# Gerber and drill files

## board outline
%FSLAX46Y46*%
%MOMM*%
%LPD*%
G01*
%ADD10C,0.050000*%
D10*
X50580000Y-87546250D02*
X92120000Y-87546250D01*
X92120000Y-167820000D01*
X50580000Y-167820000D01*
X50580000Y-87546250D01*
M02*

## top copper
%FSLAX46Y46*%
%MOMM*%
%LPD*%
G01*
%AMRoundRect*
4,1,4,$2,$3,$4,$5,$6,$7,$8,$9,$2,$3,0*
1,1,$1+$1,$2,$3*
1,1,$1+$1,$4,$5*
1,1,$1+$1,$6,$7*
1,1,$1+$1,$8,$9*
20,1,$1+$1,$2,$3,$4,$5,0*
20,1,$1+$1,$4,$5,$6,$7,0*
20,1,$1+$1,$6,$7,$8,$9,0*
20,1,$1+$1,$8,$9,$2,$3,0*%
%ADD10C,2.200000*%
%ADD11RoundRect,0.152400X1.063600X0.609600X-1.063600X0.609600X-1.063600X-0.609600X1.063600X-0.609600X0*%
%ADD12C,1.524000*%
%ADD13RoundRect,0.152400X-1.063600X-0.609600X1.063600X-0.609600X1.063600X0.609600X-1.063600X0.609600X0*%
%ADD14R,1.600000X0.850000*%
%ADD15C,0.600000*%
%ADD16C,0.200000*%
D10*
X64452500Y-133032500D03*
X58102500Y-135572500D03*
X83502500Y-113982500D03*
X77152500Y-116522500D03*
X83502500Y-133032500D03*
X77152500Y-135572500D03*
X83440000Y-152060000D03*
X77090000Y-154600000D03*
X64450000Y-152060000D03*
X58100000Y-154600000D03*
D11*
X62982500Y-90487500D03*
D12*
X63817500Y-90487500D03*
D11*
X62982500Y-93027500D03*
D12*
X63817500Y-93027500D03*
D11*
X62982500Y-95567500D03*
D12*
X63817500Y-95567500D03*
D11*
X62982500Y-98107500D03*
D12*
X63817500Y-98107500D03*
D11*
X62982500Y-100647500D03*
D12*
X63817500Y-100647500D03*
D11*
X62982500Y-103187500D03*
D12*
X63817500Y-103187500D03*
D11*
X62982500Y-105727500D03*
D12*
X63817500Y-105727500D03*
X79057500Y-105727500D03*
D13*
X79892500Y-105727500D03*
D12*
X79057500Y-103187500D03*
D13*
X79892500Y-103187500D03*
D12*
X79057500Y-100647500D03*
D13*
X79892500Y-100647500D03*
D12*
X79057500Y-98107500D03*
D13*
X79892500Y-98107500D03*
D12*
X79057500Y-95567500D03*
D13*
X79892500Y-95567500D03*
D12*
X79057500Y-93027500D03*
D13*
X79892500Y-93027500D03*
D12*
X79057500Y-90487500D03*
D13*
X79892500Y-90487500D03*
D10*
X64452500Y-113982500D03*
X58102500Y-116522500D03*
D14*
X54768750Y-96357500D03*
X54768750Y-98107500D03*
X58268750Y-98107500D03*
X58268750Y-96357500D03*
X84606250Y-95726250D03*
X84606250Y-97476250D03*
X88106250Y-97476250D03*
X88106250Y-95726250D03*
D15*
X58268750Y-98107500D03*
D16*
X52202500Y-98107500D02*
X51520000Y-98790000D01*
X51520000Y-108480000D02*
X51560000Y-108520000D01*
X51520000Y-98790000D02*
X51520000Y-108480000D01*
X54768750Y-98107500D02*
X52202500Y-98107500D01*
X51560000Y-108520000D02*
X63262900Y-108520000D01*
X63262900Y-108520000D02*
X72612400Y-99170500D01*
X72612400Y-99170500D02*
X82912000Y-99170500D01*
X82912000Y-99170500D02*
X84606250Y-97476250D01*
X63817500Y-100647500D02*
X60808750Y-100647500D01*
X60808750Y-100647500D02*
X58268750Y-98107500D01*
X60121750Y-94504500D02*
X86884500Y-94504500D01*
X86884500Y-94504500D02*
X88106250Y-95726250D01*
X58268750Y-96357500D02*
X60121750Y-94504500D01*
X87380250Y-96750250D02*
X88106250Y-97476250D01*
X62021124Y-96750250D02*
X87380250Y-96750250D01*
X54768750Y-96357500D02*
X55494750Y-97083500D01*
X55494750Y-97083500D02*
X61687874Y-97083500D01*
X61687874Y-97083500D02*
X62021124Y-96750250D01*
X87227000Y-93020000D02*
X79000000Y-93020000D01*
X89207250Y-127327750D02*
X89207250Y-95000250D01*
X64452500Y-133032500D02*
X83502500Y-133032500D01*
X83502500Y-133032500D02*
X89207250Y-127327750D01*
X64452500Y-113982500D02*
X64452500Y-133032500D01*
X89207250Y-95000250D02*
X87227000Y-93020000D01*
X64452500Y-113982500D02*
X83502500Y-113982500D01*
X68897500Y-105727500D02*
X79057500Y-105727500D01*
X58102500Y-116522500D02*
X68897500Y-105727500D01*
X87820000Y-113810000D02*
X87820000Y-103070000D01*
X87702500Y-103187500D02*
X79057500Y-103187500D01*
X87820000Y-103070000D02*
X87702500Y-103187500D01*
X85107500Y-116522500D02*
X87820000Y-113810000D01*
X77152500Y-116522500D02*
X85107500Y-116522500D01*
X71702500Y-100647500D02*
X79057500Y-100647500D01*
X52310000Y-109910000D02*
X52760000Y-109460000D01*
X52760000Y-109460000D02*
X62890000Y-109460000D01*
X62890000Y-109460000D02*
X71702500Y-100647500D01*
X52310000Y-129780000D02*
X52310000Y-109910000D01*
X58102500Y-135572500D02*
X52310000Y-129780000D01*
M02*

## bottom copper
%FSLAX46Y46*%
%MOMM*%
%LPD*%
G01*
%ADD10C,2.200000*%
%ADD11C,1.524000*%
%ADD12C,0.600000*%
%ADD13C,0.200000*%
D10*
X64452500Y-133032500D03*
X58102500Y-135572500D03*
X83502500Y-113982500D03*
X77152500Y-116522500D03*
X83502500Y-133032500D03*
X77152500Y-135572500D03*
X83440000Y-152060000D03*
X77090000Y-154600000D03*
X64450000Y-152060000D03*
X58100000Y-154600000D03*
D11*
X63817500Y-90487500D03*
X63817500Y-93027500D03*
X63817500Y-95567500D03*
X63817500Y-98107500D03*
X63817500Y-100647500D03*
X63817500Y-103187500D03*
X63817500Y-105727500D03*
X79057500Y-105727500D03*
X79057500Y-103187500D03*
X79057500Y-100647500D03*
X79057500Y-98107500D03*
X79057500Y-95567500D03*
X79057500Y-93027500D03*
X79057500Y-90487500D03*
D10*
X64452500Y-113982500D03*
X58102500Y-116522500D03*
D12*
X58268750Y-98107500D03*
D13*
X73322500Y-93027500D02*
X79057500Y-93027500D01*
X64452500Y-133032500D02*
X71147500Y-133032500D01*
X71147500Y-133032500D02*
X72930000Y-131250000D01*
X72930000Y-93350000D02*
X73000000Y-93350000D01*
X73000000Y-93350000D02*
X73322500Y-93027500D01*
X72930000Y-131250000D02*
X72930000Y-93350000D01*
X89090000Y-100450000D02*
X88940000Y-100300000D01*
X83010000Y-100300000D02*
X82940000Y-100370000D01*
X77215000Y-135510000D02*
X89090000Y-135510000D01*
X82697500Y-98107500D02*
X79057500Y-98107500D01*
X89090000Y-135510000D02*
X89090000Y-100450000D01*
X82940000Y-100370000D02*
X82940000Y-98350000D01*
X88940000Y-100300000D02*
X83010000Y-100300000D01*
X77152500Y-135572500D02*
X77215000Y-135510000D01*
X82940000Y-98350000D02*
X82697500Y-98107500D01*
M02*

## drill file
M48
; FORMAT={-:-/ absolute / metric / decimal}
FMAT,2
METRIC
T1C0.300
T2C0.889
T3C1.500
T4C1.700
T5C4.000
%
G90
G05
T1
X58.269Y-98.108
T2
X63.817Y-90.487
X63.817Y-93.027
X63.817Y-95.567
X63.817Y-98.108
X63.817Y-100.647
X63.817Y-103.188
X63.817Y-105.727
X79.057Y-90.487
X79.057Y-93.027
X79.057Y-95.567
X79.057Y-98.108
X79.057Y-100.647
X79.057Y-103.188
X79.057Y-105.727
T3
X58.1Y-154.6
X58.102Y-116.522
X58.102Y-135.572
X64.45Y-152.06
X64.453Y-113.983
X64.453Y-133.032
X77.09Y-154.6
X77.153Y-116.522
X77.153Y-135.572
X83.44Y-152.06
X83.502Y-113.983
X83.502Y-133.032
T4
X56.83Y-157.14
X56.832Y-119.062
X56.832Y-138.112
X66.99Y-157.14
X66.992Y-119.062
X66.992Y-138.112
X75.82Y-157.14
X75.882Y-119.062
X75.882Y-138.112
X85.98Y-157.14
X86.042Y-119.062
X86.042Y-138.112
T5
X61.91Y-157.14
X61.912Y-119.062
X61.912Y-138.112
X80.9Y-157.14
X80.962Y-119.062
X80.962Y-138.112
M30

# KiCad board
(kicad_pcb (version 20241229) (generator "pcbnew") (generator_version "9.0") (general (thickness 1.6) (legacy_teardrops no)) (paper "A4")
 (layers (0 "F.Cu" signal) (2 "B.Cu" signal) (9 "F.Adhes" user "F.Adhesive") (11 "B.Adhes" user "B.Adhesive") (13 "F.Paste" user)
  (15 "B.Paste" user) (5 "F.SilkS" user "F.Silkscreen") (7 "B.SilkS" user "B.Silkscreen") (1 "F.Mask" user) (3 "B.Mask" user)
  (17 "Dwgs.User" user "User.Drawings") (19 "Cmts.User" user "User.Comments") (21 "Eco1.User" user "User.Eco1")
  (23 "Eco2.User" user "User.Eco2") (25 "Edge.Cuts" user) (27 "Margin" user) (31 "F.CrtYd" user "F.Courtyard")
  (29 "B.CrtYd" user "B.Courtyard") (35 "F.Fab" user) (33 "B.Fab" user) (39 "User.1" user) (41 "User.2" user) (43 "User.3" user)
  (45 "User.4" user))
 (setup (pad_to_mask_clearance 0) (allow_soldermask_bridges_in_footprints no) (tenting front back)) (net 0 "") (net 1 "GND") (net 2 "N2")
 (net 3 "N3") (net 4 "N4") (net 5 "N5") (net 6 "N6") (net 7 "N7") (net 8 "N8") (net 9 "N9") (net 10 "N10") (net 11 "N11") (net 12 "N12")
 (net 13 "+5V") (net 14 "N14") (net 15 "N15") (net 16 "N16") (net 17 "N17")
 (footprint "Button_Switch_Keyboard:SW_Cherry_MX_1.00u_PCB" (layer "F.Cu") (at 64.4525 133.0325)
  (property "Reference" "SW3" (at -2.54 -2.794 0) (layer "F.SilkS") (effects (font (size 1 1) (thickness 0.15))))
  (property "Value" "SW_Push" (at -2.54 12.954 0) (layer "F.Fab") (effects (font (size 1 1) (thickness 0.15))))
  (pad "" np_thru_hole circle (at -7.62 5.08) (size 1.7 1.7) (drill 1.7) (layers "*.Cu" "*.Mask"))
  (pad "" np_thru_hole circle (at -2.54 5.08) (size 4 4) (drill 4) (layers "*.Cu" "*.Mask"))
  (pad "" np_thru_hole circle (at 2.54 5.08) (size 1.7 1.7) (drill 1.7) (layers "*.Cu" "*.Mask"))
  (pad "1" thru_hole circle (at 0 0) (size 2.2 2.2) (drill 1.5) (layers "*.Cu" "*.Mask") (remove_unused_layers no) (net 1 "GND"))
  (pad "2" thru_hole circle (at -6.35 2.54) (size 2.2 2.2) (drill 1.5) (layers "*.Cu" "*.Mask") (remove_unused_layers no) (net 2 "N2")))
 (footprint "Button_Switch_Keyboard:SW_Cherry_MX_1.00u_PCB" (layer "F.Cu") (at 83.5025 113.9825)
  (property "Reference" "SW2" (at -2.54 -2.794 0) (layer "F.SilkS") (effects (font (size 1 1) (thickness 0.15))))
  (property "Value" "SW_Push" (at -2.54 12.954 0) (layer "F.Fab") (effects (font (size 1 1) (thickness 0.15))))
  (pad "" np_thru_hole circle (at -7.62 5.08) (size 1.7 1.7) (drill 1.7) (layers "*.Cu" "*.Mask"))
  (pad "" np_thru_hole circle (at -2.54 5.08) (size 4 4) (drill 4) (layers "*.Cu" "*.Mask"))
  (pad "" np_thru_hole circle (at 2.54 5.08) (size 1.7 1.7) (drill 1.7) (layers "*.Cu" "*.Mask"))
  (pad "1" thru_hole circle (at 0 0) (size 2.2 2.2) (drill 1.5) (layers "*.Cu" "*.Mask") (remove_unused_layers no) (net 1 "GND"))
  (pad "2" thru_hole circle (at -6.35 2.54) (size 2.2 2.2) (drill 1.5) (layers "*.Cu" "*.Mask") (remove_unused_layers no) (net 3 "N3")))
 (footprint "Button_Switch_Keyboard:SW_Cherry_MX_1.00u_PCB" (layer "F.Cu") (at 83.5025 133.0325)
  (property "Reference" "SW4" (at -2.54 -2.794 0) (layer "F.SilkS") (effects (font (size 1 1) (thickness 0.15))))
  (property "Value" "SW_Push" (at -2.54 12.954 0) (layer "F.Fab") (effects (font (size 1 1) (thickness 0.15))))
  (pad "" np_thru_hole circle (at -7.62 5.08) (size 1.7 1.7) (drill 1.7) (layers "*.Cu" "*.Mask"))
  (pad "" np_thru_hole circle (at -2.54 5.08) (size 4 4) (drill 4) (layers "*.Cu" "*.Mask"))
  (pad "" np_thru_hole circle (at 2.54 5.08) (size 1.7 1.7) (drill 1.7) (layers "*.Cu" "*.Mask"))
  (pad "1" thru_hole circle (at 0 0) (size 2.2 2.2) (drill 1.5) (layers "*.Cu" "*.Mask") (remove_unused_layers no) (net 1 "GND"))
  (pad "2" thru_hole circle (at -6.35 2.54) (size 2.2 2.2) (drill 1.5) (layers "*.Cu" "*.Mask") (remove_unused_layers no) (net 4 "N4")))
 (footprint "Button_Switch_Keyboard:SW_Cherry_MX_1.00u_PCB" (layer "F.Cu") (at 83.44 152.06)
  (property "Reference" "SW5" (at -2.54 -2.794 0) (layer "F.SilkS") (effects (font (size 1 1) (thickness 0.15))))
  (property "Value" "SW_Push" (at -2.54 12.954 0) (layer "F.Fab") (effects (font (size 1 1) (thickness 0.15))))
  (pad "" np_thru_hole circle (at -7.62 5.08) (size 1.7 1.7) (drill 1.7) (layers "*.Cu" "*.Mask"))
  (pad "" np_thru_hole circle (at -2.54 5.08) (size 4 4) (drill 4) (layers "*.Cu" "*.Mask"))
  (pad "" np_thru_hole circle (at 2.54 5.08) (size 1.7 1.7) (drill 1.7) (layers "*.Cu" "*.Mask"))
  (pad "1" thru_hole circle (at 0 0) (size 2.2 2.2) (drill 1.5) (layers "*.Cu" "*.Mask") (remove_unused_layers no) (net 1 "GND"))
  (pad "2" thru_hole circle (at -6.35 2.54) (size 2.2 2.2) (drill 1.5) (layers "*.Cu" "*.Mask") (remove_unused_layers no) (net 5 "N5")))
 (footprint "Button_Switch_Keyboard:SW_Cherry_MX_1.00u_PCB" (layer "F.Cu") (at 64.45 152.06)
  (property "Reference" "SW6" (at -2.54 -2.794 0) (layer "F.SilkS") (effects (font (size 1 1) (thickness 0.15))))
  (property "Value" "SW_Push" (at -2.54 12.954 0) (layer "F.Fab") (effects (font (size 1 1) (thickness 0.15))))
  (pad "" np_thru_hole circle (at -7.62 5.08) (size 1.7 1.7) (drill 1.7) (layers "*.Cu" "*.Mask"))
  (pad "" np_thru_hole circle (at -2.54 5.08) (size 4 4) (drill 4) (layers "*.Cu" "*.Mask"))
  (pad "" np_thru_hole circle (at 2.54 5.08) (size 1.7 1.7) (drill 1.7) (layers "*.Cu" "*.Mask"))
  (pad "1" thru_hole circle (at 0 0) (size 2.2 2.2) (drill 1.5) (layers "*.Cu" "*.Mask") (remove_unused_layers no) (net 1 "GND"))
  (pad "2" thru_hole circle (at -6.35 2.54) (size 2.2 2.2) (drill 1.5) (layers "*.Cu" "*.Mask") (remove_unused_layers no) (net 5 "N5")))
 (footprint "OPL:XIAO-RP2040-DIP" (layer "F.Cu") (at 71.4375 98.1075)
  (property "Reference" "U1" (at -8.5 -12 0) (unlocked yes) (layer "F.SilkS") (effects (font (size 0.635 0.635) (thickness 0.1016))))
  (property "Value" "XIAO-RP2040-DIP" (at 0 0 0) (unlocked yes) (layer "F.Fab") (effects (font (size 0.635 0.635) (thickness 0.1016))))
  (pad "1" smd roundrect (at -8.455 -7.62 180) (size 2.432 1.524) (layers "F.Cu" "F.Mask") (roundrect_rratio 0.1) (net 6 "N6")
   (thermal_bridge_angle 45))
  (pad "1" thru_hole circle (at -7.62 -7.62 180) (size 1.524 1.524) (drill 0.889) (layers "*.Cu" "*.Mask") (remove_unused_layers no)
   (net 6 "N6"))
  (pad "2" smd roundrect (at -8.455 -5.08 180) (size 2.432 1.524) (layers "F.Cu" "F.Mask") (roundrect_rratio 0.1) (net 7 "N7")
   (thermal_bridge_angle 45))
  (pad "2" thru_hole circle (at -7.62 -5.08 180) (size 1.524 1.524) (drill 0.889) (layers "*.Cu" "*.Mask") (remove_unused_layers no)
   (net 7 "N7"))
  (pad "3" smd roundrect (at -8.455 -2.54 180) (size 2.432 1.524) (layers "F.Cu" "F.Mask") (roundrect_rratio 0.1) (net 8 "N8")
   (thermal_bridge_angle 45))
  (pad "3" thru_hole circle (at -7.62 -2.54 180) (size 1.524 1.524) (drill 0.889) (layers "*.Cu" "*.Mask") (remove_unused_layers no)
   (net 8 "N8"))
  (pad "4" smd roundrect (at -8.455 0 180) (size 2.432 1.524) (layers "F.Cu" "F.Mask") (roundrect_rratio 0.1) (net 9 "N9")
   (thermal_bridge_angle 45))
  (pad "4" thru_hole circle (at -7.62 0 180) (size 1.524 1.524) (drill 0.889) (layers "*.Cu" "*.Mask") (remove_unused_layers no)
   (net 9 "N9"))
  (pad "5" smd roundrect (at -8.455 2.54 180) (size 2.432 1.524) (layers "F.Cu" "F.Mask") (roundrect_rratio 0.1) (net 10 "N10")
   (thermal_bridge_angle 45))
  (pad "5" thru_hole circle (at -7.62 2.54 180) (size 1.524 1.524) (drill 0.889) (layers "*.Cu" "*.Mask") (remove_unused_layers no)
   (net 10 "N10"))
  (pad "6" smd roundrect (at -8.455 5.08 180) (size 2.432 1.524) (layers "F.Cu" "F.Mask") (roundrect_rratio 0.1) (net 5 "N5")
   (thermal_bridge_angle 45))
  (pad "6" thru_hole circle (at -7.62 5.08 180) (size 1.524 1.524) (drill 0.889) (layers "*.Cu" "*.Mask") (remove_unused_layers no)
   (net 5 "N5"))
  (pad "7" smd roundrect (at -8.455 7.62 180) (size 2.432 1.524) (layers "F.Cu" "F.Mask") (roundrect_rratio 0.1) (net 5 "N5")
   (thermal_bridge_angle 45))
  (pad "7" thru_hole circle (at -7.62 7.62 180) (size 1.524 1.524) (drill 0.889) (layers "*.Cu" "*.Mask") (remove_unused_layers no)
   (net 5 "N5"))
  (pad "8" thru_hole circle (at 7.62 7.62) (size 1.524 1.524) (drill 0.889) (layers "*.Cu" "*.Mask") (remove_unused_layers no)
   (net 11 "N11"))
  (pad "8" smd roundrect (at 8.455 7.62) (size 2.432 1.524) (layers "F.Cu" "F.Mask") (roundrect_rratio 0.1) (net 11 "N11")
   (thermal_bridge_angle 45))
  (pad "9" thru_hole circle (at 7.62 5.08) (size 1.524 1.524) (drill 0.889) (layers "*.Cu" "*.Mask") (remove_unused_layers no) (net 3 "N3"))
  (pad "9" smd roundrect (at 8.455 5.08) (size 2.432 1.524) (layers "F.Cu" "F.Mask") (roundrect_rratio 0.1) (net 3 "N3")
   (thermal_bridge_angle 45))
  (pad "10" thru_hole circle (at 7.62 2.54) (size 1.524 1.524) (drill 0.889) (layers "*.Cu" "*.Mask") (remove_unused_layers no) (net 2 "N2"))
  (pad "10" smd roundrect (at 8.455 2.54) (size 2.432 1.524) (layers "F.Cu" "F.Mask") (roundrect_rratio 0.1) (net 2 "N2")
   (thermal_bridge_angle 45))
  (pad "11" thru_hole circle (at 7.62 0) (size 1.524 1.524) (drill 0.889) (layers "*.Cu" "*.Mask") (remove_unused_layers no) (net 4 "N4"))
  (pad "11" smd roundrect (at 8.455 0) (size 2.432 1.524) (layers "F.Cu" "F.Mask") (roundrect_rratio 0.1) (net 4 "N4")
   (thermal_bridge_angle 45))
  (pad "12" thru_hole circle (at 7.62 -2.54) (size 1.524 1.524) (drill 0.889) (layers "*.Cu" "*.Mask") (remove_unused_layers no)
   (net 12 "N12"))
  (pad "12" smd roundrect (at 8.455 -2.54) (size 2.432 1.524) (layers "F.Cu" "F.Mask") (roundrect_rratio 0.1) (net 12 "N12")
   (thermal_bridge_angle 45))
  (pad "13" thru_hole circle (at 7.62 -5.08) (size 1.524 1.524) (drill 0.889) (layers "*.Cu" "*.Mask") (remove_unused_layers no)
   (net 1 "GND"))
  (pad "13" smd roundrect (at 8.455 -5.08) (size 2.432 1.524) (layers "F.Cu" "F.Mask") (roundrect_rratio 0.1) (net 1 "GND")
   (thermal_bridge_angle 45))
  (pad "14" thru_hole circle (at 7.62 -7.62) (size 1.524 1.524) (drill 0.889) (layers "*.Cu" "*.Mask") (remove_unused_layers no)
   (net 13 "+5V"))
  (pad "14" smd roundrect (at 8.455 -7.62) (size 2.432 1.524) (layers "F.Cu" "F.Mask") (roundrect_rratio 0.1) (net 13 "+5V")
   (thermal_bridge_angle 45)))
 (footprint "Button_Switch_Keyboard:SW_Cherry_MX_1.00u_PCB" (layer "F.Cu") (at 64.4525 113.9825)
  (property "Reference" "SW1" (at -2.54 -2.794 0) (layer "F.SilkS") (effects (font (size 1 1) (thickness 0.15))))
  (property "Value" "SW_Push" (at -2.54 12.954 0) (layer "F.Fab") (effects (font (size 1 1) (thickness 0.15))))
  (pad "" np_thru_hole circle (at -7.62 5.08) (size 1.7 1.7) (drill 1.7) (layers "*.Cu" "*.Mask"))
  (pad "" np_thru_hole circle (at -2.54 5.08) (size 4 4) (drill 4) (layers "*.Cu" "*.Mask"))
  (pad "" np_thru_hole circle (at 2.54 5.08) (size 1.7 1.7) (drill 1.7) (layers "*.Cu" "*.Mask"))
  (pad "1" thru_hole circle (at 0 0) (size 2.2 2.2) (drill 1.5) (layers "*.Cu" "*.Mask") (remove_unused_layers no) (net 1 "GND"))
  (pad "2" thru_hole circle (at -6.35 2.54) (size 2.2 2.2) (drill 1.5) (layers "*.Cu" "*.Mask") (remove_unused_layers no) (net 11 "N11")))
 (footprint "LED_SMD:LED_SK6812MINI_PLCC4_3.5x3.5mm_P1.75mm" (layer "F.Cu") (at 56.51875 97.2325)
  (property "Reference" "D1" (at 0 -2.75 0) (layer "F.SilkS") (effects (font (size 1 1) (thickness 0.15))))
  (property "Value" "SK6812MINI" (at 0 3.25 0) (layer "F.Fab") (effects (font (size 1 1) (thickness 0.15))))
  (pad "1" smd rect (at -1.75 -0.875) (size 1.6 0.85) (layers "F.Cu" "F.Mask" "F.Paste") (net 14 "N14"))
  (pad "2" smd rect (at -1.75 0.875) (size 1.6 0.85) (layers "F.Cu" "F.Mask" "F.Paste") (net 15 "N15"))
  (pad "3" smd rect (at 1.75 0.875) (size 1.6 0.85) (layers "F.Cu" "F.Mask" "F.Paste") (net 10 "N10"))
  (pad "4" smd rect (at 1.75 -0.875) (size 1.6 0.85) (layers "F.Cu" "F.Mask" "F.Paste") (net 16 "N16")))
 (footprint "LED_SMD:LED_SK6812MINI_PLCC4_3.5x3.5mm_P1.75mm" (layer "F.Cu") (at 86.35625 96.60125)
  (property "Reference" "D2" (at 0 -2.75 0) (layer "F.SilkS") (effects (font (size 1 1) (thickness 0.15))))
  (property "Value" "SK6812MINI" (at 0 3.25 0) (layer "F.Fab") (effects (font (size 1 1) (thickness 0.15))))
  (pad "1" smd rect (at -1.75 -0.875) (size 1.6 0.85) (layers "F.Cu" "F.Mask" "F.Paste") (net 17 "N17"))
  (pad "2" smd rect (at -1.75 0.875) (size 1.6 0.85) (layers "F.Cu" "F.Mask" "F.Paste") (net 15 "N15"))
  (pad "3" smd rect (at 1.75 0.875) (size 1.6 0.85) (layers "F.Cu" "F.Mask" "F.Paste") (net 14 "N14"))
  (pad "4" smd rect (at 1.75 -0.875) (size 1.6 0.85) (layers "F.Cu" "F.Mask" "F.Paste") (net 16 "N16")))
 (gr_rect (start 50.58 87.54625) (end 92.12 167.82) (stroke (width 0.05) (type default)) (fill no) (layer "Edge.Cuts"))
 (segment (start 52.2025 98.1075) (end 51.52 98.79) (width 0.2) (layer "F.Cu") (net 15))
 (segment (start 51.52 108.48) (end 51.56 108.52) (width 0.2) (layer "F.Cu") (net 15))
 (segment (start 51.52 98.79) (end 51.52 108.48) (width 0.2) (layer "F.Cu") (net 15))
 (segment (start 54.76875 98.1075) (end 52.2025 98.1075) (width 0.2) (layer "F.Cu") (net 15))
 (segment (start 51.56 108.52) (end 63.2629 108.52) (width 0.2) (layer "F.Cu") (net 15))
 (segment (start 63.2629 108.52) (end 72.6124 99.1705) (width 0.2) (layer "F.Cu") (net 15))
 (segment (start 72.6124 99.1705) (end 82.912 99.1705) (width 0.2) (layer "F.Cu") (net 15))
 (segment (start 82.912 99.1705) (end 84.60625 97.47625) (width 0.2) (layer "F.Cu") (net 15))
 (segment (start 63.8175 100.6475) (end 60.80875 100.6475) (width 0.2) (layer "F.Cu") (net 10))
 (segment (start 60.80875 100.6475) (end 58.26875 98.1075) (width 0.2) (layer "F.Cu") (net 10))
 (via (at 58.26875 98.1075) (size 0.6) (drill 0.3) (layers "F.Cu" "B.Cu") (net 10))
 (segment (start 60.12175 94.5045) (end 86.8845 94.5045) (width 0.2) (layer "F.Cu") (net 16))
 (segment (start 86.8845 94.5045) (end 88.10625 95.72625) (width 0.2) (layer "F.Cu") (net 16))
 (segment (start 58.26875 96.3575) (end 60.12175 94.5045) (width 0.2) (layer "F.Cu") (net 16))
 (segment (start 87.38025 96.75025) (end 88.10625 97.47625) (width 0.2) (layer "F.Cu") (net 14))
 (segment (start 62.021124 96.75025) (end 87.38025 96.75025) (width 0.2) (layer "F.Cu") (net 14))
 (segment (start 54.76875 96.3575) (end 55.49475 97.0835) (width 0.2) (layer "F.Cu") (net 14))
 (segment (start 55.49475 97.0835) (end 61.687874 97.0835) (width 0.2) (layer "F.Cu") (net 14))
 (segment (start 61.687874 97.0835) (end 62.021124 96.75025) (width 0.2) (layer "F.Cu") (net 14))
 (segment (start 87.227 93.02) (end 79 93.02) (width 0.2) (layer "F.Cu") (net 1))
 (segment (start 89.20725 127.32775) (end 89.20725 95.00025) (width 0.2) (layer "F.Cu") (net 1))
 (segment (start 64.4525 133.0325) (end 83.5025 133.0325) (width 0.2) (layer "F.Cu") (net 1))
 (segment (start 83.5025 133.0325) (end 89.20725 127.32775) (width 0.2) (layer "F.Cu") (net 1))
 (segment (start 64.4525 113.9825) (end 64.4525 133.0325) (width 0.2) (layer "F.Cu") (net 1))
 (segment (start 89.20725 95.00025) (end 87.227 93.02) (width 0.2) (layer "F.Cu") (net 1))
 (segment (start 64.4525 113.9825) (end 83.5025 113.9825) (width 0.2) (layer "F.Cu") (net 1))
 (segment (start 73.3225 93.0275) (end 79.0575 93.0275) (width 0.2) (layer "B.Cu") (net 1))
 (segment (start 64.4525 133.0325) (end 71.1475 133.0325) (width 0.2) (layer "B.Cu") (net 1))
 (segment (start 71.1475 133.0325) (end 72.93 131.25) (width 0.2) (layer "B.Cu") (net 1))
 (segment (start 72.93 93.35) (end 73 93.35) (width 0.2) (layer "B.Cu") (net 1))
 (segment (start 73 93.35) (end 73.3225 93.0275) (width 0.2) (layer "B.Cu") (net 1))
 (segment (start 72.93 131.25) (end 72.93 93.35) (width 0.2) (layer "B.Cu") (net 1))
 (segment (start 68.8975 105.7275) (end 79.0575 105.7275) (width 0.2) (layer "F.Cu") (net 11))
 (segment (start 58.1025 116.5225) (end 68.8975 105.7275) (width 0.2) (layer "F.Cu") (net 11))
 (segment (start 87.82 113.81) (end 87.82 103.07) (width 0.2) (layer "F.Cu") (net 3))
 (segment (start 87.7025 103.1875) (end 79.0575 103.1875) (width 0.2) (layer "F.Cu") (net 3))
 (segment (start 87.82 103.07) (end 87.7025 103.1875) (width 0.2) (layer "F.Cu") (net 3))
 (segment (start 85.1075 116.5225) (end 87.82 113.81) (width 0.2) (layer "F.Cu") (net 3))
 (segment (start 77.1525 116.5225) (end 85.1075 116.5225) (width 0.2) (layer "F.Cu") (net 3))
 (segment (start 71.7025 100.6475) (end 79.0575 100.6475) (width 0.2) (layer "F.Cu") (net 2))
 (segment (start 52.31 109.91) (end 52.76 109.46) (width 0.2) (layer "F.Cu") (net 2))
 (segment (start 52.76 109.46) (end 62.89 109.46) (width 0.2) (layer "F.Cu") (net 2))
 (segment (start 62.89 109.46) (end 71.7025 100.6475) (width 0.2) (layer "F.Cu") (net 2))
 (segment (start 52.31 129.78) (end 52.31 109.91) (width 0.2) (layer "F.Cu") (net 2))
 (segment (start 58.1025 135.5725) (end 52.31 129.78) (width 0.2) (layer "F.Cu") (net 2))
 (segment (start 89.09 100.45) (end 88.94 100.3) (width 0.2) (layer "B.Cu") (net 4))
 (segment (start 83.01 100.3) (end 82.94 100.37) (width 0.2) (layer "B.Cu") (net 4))
 (segment (start 77.215 135.51) (end 89.09 135.51) (width 0.2) (layer "B.Cu") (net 4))
 (segment (start 82.6975 98.1075) (end 79.0575 98.1075) (width 0.2) (layer "B.Cu") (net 4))
 (segment (start 89.09 135.51) (end 89.09 100.45) (width 0.2) (layer "B.Cu") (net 4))
 (segment (start 82.94 100.37) (end 82.94 98.35) (width 0.2) (layer "B.Cu") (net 4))
 (segment (start 88.94 100.3) (end 83.01 100.3) (width 0.2) (layer "B.Cu") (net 4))
 (segment (start 77.1525 135.5725) (end 77.215 135.51) (width 0.2) (layer "B.Cu") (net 4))
 (segment (start 82.94 98.35) (end 82.6975 98.1075) (width 0.2) (layer "B.Cu") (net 4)))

